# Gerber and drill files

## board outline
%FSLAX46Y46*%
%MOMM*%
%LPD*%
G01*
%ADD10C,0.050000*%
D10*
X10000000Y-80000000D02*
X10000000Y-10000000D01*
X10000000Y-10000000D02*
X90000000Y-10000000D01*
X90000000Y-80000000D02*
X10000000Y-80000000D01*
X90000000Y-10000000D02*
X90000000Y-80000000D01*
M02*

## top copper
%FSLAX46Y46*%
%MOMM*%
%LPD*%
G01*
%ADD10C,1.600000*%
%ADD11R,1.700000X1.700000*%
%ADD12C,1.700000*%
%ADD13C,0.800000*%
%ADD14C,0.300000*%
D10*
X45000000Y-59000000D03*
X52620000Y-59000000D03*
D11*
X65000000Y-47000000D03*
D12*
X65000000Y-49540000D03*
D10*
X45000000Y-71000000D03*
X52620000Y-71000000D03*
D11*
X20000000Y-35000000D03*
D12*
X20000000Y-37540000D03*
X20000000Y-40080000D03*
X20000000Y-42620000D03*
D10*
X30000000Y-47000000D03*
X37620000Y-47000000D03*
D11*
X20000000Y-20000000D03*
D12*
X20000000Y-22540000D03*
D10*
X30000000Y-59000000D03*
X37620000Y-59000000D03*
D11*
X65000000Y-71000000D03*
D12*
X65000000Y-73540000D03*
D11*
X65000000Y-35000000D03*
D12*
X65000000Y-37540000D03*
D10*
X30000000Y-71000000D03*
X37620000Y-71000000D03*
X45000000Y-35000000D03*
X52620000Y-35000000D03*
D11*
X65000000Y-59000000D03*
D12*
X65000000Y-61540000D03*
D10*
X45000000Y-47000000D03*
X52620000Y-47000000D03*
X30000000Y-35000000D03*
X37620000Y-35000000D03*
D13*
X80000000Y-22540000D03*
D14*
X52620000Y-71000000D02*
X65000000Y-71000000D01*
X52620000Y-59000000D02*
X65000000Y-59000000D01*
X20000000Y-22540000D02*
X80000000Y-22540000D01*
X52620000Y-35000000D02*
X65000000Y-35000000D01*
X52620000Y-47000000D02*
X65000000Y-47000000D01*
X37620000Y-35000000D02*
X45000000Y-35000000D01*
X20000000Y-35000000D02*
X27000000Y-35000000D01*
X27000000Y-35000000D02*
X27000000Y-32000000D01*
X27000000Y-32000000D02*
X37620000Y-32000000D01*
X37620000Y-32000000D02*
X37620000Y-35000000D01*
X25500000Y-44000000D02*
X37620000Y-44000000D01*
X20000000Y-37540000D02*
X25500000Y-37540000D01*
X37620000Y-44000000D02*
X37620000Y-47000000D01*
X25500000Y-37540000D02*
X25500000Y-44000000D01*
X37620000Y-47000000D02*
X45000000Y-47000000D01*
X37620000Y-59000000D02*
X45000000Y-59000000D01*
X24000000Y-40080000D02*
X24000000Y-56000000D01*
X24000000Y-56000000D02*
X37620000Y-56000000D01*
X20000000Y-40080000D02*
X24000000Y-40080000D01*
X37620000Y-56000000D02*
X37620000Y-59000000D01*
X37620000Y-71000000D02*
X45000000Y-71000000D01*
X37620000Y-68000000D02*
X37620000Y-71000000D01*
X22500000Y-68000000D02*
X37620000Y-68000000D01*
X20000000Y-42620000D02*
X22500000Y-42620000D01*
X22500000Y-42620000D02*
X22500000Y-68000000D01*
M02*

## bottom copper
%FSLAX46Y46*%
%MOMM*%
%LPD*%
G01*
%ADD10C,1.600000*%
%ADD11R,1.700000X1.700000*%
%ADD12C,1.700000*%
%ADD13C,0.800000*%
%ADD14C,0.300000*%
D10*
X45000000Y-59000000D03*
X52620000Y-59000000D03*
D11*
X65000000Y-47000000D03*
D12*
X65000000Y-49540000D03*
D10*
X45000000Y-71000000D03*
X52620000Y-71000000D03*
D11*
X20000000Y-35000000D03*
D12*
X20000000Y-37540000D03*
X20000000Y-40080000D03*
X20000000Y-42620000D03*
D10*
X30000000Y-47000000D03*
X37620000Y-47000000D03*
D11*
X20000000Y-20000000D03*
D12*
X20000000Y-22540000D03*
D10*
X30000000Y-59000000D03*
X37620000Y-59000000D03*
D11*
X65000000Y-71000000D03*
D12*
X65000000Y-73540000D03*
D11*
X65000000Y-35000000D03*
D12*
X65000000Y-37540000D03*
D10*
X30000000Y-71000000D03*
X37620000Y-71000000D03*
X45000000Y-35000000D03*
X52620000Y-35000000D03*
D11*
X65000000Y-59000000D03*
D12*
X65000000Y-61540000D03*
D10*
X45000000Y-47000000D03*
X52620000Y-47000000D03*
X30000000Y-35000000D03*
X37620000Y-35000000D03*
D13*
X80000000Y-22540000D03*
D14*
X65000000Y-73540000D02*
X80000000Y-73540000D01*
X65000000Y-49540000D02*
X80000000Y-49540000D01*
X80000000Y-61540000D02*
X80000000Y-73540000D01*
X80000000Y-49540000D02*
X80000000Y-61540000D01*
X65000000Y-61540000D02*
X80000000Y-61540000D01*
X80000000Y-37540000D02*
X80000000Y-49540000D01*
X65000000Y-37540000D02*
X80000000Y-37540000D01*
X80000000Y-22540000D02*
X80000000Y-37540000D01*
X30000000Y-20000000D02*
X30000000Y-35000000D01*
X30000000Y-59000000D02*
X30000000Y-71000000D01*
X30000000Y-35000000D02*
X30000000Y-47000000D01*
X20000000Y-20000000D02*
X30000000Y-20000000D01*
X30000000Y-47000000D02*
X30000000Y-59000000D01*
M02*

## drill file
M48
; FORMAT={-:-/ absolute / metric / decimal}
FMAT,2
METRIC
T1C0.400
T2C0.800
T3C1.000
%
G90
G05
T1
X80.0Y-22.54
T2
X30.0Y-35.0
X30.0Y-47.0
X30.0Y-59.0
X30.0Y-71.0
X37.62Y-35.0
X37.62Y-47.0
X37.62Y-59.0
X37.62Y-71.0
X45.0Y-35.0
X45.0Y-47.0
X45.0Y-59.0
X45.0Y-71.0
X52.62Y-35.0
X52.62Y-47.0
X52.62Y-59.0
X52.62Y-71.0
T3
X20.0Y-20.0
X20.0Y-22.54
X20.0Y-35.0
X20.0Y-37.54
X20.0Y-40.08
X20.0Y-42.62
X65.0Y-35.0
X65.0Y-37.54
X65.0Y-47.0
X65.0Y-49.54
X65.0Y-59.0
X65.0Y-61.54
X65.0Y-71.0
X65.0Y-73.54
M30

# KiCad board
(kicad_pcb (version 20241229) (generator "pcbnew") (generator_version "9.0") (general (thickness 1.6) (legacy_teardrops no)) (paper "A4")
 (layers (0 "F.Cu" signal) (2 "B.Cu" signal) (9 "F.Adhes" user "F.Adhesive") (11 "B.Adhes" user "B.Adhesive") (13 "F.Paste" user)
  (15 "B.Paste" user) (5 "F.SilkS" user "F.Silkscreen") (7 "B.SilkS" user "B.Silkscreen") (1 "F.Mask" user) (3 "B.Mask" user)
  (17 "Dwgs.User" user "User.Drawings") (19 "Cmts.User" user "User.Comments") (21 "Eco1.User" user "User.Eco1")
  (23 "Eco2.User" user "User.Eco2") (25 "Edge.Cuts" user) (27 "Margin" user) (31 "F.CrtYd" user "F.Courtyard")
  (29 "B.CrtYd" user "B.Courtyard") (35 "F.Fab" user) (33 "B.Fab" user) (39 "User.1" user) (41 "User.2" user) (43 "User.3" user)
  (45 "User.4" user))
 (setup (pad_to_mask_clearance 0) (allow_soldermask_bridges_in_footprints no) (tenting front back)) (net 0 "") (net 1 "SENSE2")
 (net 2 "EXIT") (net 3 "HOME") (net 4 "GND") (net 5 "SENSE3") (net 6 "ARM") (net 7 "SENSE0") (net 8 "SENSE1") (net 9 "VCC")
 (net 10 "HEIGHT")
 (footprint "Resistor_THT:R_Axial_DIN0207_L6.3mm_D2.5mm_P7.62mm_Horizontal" (layer "F.Cu") (at 45 59)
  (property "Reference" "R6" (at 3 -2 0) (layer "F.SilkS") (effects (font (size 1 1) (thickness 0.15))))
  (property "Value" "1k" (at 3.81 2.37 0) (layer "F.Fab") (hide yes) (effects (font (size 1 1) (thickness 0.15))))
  (pad "1" thru_hole circle (at 0 0) (size 1.6 1.6) (drill 0.8) (layers "*.Cu" "*.Mask") (remove_unused_layers no) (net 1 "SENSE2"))
  (pad "2" thru_hole circle (at 7.62 0) (size 1.6 1.6) (drill 0.8) (layers "*.Cu" "*.Mask") (remove_unused_layers no) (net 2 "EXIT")))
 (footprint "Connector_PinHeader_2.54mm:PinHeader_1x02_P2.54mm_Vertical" (layer "F.Cu") (at 65 47)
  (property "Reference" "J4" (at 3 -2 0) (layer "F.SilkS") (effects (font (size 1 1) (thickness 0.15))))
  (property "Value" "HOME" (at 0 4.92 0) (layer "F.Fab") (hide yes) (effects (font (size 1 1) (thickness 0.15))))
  (pad "1" thru_hole rect (at 0 0) (size 1.7 1.7) (drill 1) (layers "*.Cu" "*.Mask") (remove_unused_layers no) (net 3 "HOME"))
  (pad "2" thru_hole circle (at 0 2.54) (size 1.7 1.7) (drill 1) (layers "*.Cu" "*.Mask") (remove_unused_layers no) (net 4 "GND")))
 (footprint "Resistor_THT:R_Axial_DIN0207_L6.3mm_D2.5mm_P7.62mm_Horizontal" (layer "F.Cu") (at 45 71)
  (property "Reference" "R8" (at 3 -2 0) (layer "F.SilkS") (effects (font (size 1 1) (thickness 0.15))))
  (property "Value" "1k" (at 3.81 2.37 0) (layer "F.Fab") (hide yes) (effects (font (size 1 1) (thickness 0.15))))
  (pad "1" thru_hole circle (at 0 0) (size 1.6 1.6) (drill 0.8) (layers "*.Cu" "*.Mask") (remove_unused_layers no) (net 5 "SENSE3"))
  (pad "2" thru_hole circle (at 7.62 0) (size 1.6 1.6) (drill 0.8) (layers "*.Cu" "*.Mask") (remove_unused_layers no) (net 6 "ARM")))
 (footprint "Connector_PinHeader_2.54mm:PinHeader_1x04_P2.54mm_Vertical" (layer "F.Cu") (at 20 35)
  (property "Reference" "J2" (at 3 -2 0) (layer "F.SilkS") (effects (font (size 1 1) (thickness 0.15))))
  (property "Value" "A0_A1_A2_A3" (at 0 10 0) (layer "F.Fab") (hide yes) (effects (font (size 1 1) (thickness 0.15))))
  (pad "1" thru_hole rect (at 0 0) (size 1.7 1.7) (drill 1) (layers "*.Cu" "*.Mask") (remove_unused_layers no) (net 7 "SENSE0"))
  (pad "2" thru_hole circle (at 0 2.54) (size 1.7 1.7) (drill 1) (layers "*.Cu" "*.Mask") (remove_unused_layers no) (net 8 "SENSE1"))
  (pad "3" thru_hole circle (at 0 5.08) (size 1.7 1.7) (drill 1) (layers "*.Cu" "*.Mask") (remove_unused_layers no) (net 1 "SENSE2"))
  (pad "4" thru_hole circle (at 0 7.62) (size 1.7 1.7) (drill 1) (layers "*.Cu" "*.Mask") (remove_unused_layers no) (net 5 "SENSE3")))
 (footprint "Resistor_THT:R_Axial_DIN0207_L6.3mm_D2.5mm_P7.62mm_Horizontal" (layer "F.Cu") (at 30 47)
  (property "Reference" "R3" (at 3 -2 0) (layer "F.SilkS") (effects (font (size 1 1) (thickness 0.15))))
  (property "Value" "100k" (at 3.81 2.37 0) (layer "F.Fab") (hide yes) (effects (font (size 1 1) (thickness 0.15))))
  (pad "1" thru_hole circle (at 0 0) (size 1.6 1.6) (drill 0.8) (layers "*.Cu" "*.Mask") (remove_unused_layers no) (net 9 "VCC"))
  (pad "2" thru_hole circle (at 7.62 0) (size 1.6 1.6) (drill 0.8) (layers "*.Cu" "*.Mask") (remove_unused_layers no) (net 8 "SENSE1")))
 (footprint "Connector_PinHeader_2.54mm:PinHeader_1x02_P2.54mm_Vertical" (layer "F.Cu") (at 20 20)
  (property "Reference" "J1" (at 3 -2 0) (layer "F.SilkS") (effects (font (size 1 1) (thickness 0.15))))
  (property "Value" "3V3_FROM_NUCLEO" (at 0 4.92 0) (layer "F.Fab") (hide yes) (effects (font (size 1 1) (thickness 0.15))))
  (pad "1" thru_hole rect (at 0 0) (size 1.7 1.7) (drill 1) (layers "*.Cu" "*.Mask") (remove_unused_layers no) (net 9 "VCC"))
  (pad "2" thru_hole circle (at 0 2.54) (size 1.7 1.7) (drill 1) (layers "*.Cu" "*.Mask") (remove_unused_layers no) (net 4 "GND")))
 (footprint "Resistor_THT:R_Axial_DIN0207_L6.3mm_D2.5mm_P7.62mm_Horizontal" (layer "F.Cu") (at 30 59)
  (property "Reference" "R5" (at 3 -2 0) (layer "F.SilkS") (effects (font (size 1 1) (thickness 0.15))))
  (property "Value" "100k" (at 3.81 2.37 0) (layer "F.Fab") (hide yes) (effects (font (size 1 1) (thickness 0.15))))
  (pad "1" thru_hole circle (at 0 0) (size 1.6 1.6) (drill 0.8) (layers "*.Cu" "*.Mask") (remove_unused_layers no) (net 9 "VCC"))
  (pad "2" thru_hole circle (at 7.62 0) (size 1.6 1.6) (drill 0.8) (layers "*.Cu" "*.Mask") (remove_unused_layers no) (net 1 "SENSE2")))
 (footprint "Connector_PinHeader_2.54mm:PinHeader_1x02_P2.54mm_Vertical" (layer "F.Cu") (at 65 71)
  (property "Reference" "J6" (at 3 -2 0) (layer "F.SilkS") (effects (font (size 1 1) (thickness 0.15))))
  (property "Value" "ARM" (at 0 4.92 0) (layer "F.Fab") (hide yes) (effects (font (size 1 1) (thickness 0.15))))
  (pad "1" thru_hole rect (at 0 0) (size 1.7 1.7) (drill 1) (layers "*.Cu" "*.Mask") (remove_unused_layers no) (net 6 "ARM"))
  (pad "2" thru_hole circle (at 0 2.54) (size 1.7 1.7) (drill 1) (layers "*.Cu" "*.Mask") (remove_unused_layers no) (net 4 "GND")))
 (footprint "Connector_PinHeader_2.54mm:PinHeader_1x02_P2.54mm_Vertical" (layer "F.Cu") (at 65 35)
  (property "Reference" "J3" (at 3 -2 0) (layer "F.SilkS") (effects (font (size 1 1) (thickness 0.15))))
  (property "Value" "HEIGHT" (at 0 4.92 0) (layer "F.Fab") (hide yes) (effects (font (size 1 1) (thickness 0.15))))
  (pad "1" thru_hole rect (at 0 0) (size 1.7 1.7) (drill 1) (layers "*.Cu" "*.Mask") (remove_unused_layers no) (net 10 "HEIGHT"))
  (pad "2" thru_hole circle (at 0 2.54) (size 1.7 1.7) (drill 1) (layers "*.Cu" "*.Mask") (remove_unused_layers no) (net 4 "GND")))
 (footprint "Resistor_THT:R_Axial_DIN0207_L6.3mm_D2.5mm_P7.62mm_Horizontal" (layer "F.Cu") (at 30 71)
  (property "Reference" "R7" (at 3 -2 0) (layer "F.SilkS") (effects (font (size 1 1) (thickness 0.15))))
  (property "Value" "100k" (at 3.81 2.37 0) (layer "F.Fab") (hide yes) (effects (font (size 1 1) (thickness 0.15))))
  (pad "1" thru_hole circle (at 0 0) (size 1.6 1.6) (drill 0.8) (layers "*.Cu" "*.Mask") (remove_unused_layers no) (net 9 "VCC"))
  (pad "2" thru_hole circle (at 7.62 0) (size 1.6 1.6) (drill 0.8) (layers "*.Cu" "*.Mask") (remove_unused_layers no) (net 5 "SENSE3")))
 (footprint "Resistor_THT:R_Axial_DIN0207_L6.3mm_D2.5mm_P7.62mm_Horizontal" (layer "F.Cu") (at 45 35)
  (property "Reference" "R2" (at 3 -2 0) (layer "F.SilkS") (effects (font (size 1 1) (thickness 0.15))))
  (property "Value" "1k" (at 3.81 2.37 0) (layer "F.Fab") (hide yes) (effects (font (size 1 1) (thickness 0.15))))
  (pad "1" thru_hole circle (at 0 0) (size 1.6 1.6) (drill 0.8) (layers "*.Cu" "*.Mask") (remove_unused_layers no) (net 7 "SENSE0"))
  (pad "2" thru_hole circle (at 7.62 0) (size 1.6 1.6) (drill 0.8) (layers "*.Cu" "*.Mask") (remove_unused_layers no) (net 10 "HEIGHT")))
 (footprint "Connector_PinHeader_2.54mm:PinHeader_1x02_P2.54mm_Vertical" (layer "F.Cu") (at 65 59)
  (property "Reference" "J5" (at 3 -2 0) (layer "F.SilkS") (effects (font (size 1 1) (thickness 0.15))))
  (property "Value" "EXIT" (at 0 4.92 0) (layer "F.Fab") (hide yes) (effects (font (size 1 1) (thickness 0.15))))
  (pad "1" thru_hole rect (at 0 0) (size 1.7 1.7) (drill 1) (layers "*.Cu" "*.Mask") (remove_unused_layers no) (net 2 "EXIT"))
  (pad "2" thru_hole circle (at 0 2.54) (size 1.7 1.7) (drill 1) (layers "*.Cu" "*.Mask") (remove_unused_layers no) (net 4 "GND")))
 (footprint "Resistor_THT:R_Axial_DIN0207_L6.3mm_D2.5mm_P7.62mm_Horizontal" (layer "F.Cu") (at 45 47)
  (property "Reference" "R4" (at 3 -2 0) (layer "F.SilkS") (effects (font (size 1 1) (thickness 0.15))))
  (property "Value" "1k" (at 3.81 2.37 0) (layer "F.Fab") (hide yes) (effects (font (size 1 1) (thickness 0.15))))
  (pad "1" thru_hole circle (at 0 0) (size 1.6 1.6) (drill 0.8) (layers "*.Cu" "*.Mask") (remove_unused_layers no) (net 8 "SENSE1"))
  (pad "2" thru_hole circle (at 7.62 0) (size 1.6 1.6) (drill 0.8) (layers "*.Cu" "*.Mask") (remove_unused_layers no) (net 3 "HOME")))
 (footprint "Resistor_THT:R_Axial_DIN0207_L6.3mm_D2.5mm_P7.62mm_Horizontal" (layer "F.Cu") (at 30 35)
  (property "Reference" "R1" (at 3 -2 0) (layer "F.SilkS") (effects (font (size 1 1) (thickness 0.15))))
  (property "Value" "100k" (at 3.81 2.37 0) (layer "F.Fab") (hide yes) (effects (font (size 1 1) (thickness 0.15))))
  (pad "1" thru_hole circle (at 0 0) (size 1.6 1.6) (drill 0.8) (layers "*.Cu" "*.Mask") (remove_unused_layers no) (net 9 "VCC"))
  (pad "2" thru_hole circle (at 7.62 0) (size 1.6 1.6) (drill 0.8) (layers "*.Cu" "*.Mask") (remove_unused_layers no) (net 7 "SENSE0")))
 (gr_line (start 10 80) (end 10 10) (stroke (width 0.05) (type default)) (layer "Edge.Cuts"))
 (gr_line (start 10 10) (end 90 10) (stroke (width 0.05) (type default)) (layer "Edge.Cuts"))
 (gr_line (start 90 80) (end 10 80) (stroke (width 0.05) (type default)) (layer "Edge.Cuts"))
 (gr_line (start 90 10) (end 90 80) (stroke (width 0.05) (type default)) (layer "Edge.Cuts"))
 (segment (start 52.62 71) (end 65 71) (width 0.3) (layer "F.Cu") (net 6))
 (segment (start 52.62 59) (end 65 59) (width 0.3) (layer "F.Cu") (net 2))
 (segment (start 20 22.54) (end 80 22.54) (width 0.3) (layer "F.Cu") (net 4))
 (via (at 80 22.54) (size 0.8) (drill 0.4) (layers "F.Cu" "B.Cu") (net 4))
 (segment (start 65 73.54) (end 80 73.54) (width 0.3) (layer "B.Cu") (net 4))
 (segment (start 65 49.54) (end 80 49.54) (width 0.3) (layer "B.Cu") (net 4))
 (segment (start 80 61.54) (end 80 73.54) (width 0.3) (layer "B.Cu") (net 4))
 (segment (start 80 49.54) (end 80 61.54) (width 0.3) (layer "B.Cu") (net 4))
 (segment (start 65 61.54) (end 80 61.54) (width 0.3) (layer "B.Cu") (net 4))
 (segment (start 80 37.54) (end 80 49.54) (width 0.3) (layer "B.Cu") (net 4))
 (segment (start 65 37.54) (end 80 37.54) (width 0.3) (layer "B.Cu") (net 4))
 (segment (start 80 22.54) (end 80 37.54) (width 0.3) (layer "B.Cu") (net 4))
 (segment (start 52.62 35) (end 65 35) (width 0.3) (layer "F.Cu") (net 10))
 (segment (start 52.62 47) (end 65 47) (width 0.3) (layer "F.Cu") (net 3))
 (segment (start 37.62 35) (end 45 35) (width 0.3) (layer "F.Cu") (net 7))
 (segment (start 20 35) (end 27 35) (width 0.3) (layer "F.Cu") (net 7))
 (segment (start 27 35) (end 27 32) (width 0.3) (layer "F.Cu") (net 7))
 (segment (start 27 32) (end 37.62 32) (width 0.3) (layer "F.Cu") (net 7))
 (segment (start 37.62 32) (end 37.62 35) (width 0.3) (layer "F.Cu") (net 7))
 (segment (start 25.5 44) (end 37.62 44) (width 0.3) (layer "F.Cu") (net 8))
 (segment (start 20 37.54) (end 25.5 37.54) (width 0.3) (layer "F.Cu") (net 8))
 (segment (start 37.62 44) (end 37.62 47) (width 0.3) (layer "F.Cu") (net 8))
 (segment (start 25.5 37.54) (end 25.5 44) (width 0.3) (layer "F.Cu") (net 8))
 (segment (start 37.62 47) (end 45 47) (width 0.3) (layer "F.Cu") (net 8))
 (segment (start 37.62 59) (end 45 59) (width 0.3) (layer "F.Cu") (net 1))
 (segment (start 24 40.08) (end 24 56) (width 0.3) (layer "F.Cu") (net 1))
 (segment (start 24 56) (end 37.62 56) (width 0.3) (layer "F.Cu") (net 1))
 (segment (start 20 40.08) (end 24 40.08) (width 0.3) (layer "F.Cu") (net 1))
 (segment (start 37.62 56) (end 37.62 59) (width 0.3) (layer "F.Cu") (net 1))
 (segment (start 37.62 71) (end 45 71) (width 0.3) (layer "F.Cu") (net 5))
 (segment (start 37.62 68) (end 37.62 71) (width 0.3) (layer "F.Cu") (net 5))
 (segment (start 22.5 68) (end 37.62 68) (width 0.3) (layer "F.Cu") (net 5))
 (segment (start 20 42.62) (end 22.5 42.62) (width 0.3) (layer "F.Cu") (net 5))
 (segment (start 22.5 42.62) (end 22.5 68) (width 0.3) (layer "F.Cu") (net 5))
 (segment (start 30 20) (end 30 35) (width 0.3) (layer "B.Cu") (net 9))
 (segment (start 30 59) (end 30 71) (width 0.3) (layer "B.Cu") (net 9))
 (segment (start 30 35) (end 30 47) (width 0.3) (layer "B.Cu") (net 9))
 (segment (start 20 20) (end 30 20) (width 0.3) (layer "B.Cu") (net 9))
 (segment (start 30 47) (end 30 59) (width 0.3) (layer "B.Cu") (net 9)))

